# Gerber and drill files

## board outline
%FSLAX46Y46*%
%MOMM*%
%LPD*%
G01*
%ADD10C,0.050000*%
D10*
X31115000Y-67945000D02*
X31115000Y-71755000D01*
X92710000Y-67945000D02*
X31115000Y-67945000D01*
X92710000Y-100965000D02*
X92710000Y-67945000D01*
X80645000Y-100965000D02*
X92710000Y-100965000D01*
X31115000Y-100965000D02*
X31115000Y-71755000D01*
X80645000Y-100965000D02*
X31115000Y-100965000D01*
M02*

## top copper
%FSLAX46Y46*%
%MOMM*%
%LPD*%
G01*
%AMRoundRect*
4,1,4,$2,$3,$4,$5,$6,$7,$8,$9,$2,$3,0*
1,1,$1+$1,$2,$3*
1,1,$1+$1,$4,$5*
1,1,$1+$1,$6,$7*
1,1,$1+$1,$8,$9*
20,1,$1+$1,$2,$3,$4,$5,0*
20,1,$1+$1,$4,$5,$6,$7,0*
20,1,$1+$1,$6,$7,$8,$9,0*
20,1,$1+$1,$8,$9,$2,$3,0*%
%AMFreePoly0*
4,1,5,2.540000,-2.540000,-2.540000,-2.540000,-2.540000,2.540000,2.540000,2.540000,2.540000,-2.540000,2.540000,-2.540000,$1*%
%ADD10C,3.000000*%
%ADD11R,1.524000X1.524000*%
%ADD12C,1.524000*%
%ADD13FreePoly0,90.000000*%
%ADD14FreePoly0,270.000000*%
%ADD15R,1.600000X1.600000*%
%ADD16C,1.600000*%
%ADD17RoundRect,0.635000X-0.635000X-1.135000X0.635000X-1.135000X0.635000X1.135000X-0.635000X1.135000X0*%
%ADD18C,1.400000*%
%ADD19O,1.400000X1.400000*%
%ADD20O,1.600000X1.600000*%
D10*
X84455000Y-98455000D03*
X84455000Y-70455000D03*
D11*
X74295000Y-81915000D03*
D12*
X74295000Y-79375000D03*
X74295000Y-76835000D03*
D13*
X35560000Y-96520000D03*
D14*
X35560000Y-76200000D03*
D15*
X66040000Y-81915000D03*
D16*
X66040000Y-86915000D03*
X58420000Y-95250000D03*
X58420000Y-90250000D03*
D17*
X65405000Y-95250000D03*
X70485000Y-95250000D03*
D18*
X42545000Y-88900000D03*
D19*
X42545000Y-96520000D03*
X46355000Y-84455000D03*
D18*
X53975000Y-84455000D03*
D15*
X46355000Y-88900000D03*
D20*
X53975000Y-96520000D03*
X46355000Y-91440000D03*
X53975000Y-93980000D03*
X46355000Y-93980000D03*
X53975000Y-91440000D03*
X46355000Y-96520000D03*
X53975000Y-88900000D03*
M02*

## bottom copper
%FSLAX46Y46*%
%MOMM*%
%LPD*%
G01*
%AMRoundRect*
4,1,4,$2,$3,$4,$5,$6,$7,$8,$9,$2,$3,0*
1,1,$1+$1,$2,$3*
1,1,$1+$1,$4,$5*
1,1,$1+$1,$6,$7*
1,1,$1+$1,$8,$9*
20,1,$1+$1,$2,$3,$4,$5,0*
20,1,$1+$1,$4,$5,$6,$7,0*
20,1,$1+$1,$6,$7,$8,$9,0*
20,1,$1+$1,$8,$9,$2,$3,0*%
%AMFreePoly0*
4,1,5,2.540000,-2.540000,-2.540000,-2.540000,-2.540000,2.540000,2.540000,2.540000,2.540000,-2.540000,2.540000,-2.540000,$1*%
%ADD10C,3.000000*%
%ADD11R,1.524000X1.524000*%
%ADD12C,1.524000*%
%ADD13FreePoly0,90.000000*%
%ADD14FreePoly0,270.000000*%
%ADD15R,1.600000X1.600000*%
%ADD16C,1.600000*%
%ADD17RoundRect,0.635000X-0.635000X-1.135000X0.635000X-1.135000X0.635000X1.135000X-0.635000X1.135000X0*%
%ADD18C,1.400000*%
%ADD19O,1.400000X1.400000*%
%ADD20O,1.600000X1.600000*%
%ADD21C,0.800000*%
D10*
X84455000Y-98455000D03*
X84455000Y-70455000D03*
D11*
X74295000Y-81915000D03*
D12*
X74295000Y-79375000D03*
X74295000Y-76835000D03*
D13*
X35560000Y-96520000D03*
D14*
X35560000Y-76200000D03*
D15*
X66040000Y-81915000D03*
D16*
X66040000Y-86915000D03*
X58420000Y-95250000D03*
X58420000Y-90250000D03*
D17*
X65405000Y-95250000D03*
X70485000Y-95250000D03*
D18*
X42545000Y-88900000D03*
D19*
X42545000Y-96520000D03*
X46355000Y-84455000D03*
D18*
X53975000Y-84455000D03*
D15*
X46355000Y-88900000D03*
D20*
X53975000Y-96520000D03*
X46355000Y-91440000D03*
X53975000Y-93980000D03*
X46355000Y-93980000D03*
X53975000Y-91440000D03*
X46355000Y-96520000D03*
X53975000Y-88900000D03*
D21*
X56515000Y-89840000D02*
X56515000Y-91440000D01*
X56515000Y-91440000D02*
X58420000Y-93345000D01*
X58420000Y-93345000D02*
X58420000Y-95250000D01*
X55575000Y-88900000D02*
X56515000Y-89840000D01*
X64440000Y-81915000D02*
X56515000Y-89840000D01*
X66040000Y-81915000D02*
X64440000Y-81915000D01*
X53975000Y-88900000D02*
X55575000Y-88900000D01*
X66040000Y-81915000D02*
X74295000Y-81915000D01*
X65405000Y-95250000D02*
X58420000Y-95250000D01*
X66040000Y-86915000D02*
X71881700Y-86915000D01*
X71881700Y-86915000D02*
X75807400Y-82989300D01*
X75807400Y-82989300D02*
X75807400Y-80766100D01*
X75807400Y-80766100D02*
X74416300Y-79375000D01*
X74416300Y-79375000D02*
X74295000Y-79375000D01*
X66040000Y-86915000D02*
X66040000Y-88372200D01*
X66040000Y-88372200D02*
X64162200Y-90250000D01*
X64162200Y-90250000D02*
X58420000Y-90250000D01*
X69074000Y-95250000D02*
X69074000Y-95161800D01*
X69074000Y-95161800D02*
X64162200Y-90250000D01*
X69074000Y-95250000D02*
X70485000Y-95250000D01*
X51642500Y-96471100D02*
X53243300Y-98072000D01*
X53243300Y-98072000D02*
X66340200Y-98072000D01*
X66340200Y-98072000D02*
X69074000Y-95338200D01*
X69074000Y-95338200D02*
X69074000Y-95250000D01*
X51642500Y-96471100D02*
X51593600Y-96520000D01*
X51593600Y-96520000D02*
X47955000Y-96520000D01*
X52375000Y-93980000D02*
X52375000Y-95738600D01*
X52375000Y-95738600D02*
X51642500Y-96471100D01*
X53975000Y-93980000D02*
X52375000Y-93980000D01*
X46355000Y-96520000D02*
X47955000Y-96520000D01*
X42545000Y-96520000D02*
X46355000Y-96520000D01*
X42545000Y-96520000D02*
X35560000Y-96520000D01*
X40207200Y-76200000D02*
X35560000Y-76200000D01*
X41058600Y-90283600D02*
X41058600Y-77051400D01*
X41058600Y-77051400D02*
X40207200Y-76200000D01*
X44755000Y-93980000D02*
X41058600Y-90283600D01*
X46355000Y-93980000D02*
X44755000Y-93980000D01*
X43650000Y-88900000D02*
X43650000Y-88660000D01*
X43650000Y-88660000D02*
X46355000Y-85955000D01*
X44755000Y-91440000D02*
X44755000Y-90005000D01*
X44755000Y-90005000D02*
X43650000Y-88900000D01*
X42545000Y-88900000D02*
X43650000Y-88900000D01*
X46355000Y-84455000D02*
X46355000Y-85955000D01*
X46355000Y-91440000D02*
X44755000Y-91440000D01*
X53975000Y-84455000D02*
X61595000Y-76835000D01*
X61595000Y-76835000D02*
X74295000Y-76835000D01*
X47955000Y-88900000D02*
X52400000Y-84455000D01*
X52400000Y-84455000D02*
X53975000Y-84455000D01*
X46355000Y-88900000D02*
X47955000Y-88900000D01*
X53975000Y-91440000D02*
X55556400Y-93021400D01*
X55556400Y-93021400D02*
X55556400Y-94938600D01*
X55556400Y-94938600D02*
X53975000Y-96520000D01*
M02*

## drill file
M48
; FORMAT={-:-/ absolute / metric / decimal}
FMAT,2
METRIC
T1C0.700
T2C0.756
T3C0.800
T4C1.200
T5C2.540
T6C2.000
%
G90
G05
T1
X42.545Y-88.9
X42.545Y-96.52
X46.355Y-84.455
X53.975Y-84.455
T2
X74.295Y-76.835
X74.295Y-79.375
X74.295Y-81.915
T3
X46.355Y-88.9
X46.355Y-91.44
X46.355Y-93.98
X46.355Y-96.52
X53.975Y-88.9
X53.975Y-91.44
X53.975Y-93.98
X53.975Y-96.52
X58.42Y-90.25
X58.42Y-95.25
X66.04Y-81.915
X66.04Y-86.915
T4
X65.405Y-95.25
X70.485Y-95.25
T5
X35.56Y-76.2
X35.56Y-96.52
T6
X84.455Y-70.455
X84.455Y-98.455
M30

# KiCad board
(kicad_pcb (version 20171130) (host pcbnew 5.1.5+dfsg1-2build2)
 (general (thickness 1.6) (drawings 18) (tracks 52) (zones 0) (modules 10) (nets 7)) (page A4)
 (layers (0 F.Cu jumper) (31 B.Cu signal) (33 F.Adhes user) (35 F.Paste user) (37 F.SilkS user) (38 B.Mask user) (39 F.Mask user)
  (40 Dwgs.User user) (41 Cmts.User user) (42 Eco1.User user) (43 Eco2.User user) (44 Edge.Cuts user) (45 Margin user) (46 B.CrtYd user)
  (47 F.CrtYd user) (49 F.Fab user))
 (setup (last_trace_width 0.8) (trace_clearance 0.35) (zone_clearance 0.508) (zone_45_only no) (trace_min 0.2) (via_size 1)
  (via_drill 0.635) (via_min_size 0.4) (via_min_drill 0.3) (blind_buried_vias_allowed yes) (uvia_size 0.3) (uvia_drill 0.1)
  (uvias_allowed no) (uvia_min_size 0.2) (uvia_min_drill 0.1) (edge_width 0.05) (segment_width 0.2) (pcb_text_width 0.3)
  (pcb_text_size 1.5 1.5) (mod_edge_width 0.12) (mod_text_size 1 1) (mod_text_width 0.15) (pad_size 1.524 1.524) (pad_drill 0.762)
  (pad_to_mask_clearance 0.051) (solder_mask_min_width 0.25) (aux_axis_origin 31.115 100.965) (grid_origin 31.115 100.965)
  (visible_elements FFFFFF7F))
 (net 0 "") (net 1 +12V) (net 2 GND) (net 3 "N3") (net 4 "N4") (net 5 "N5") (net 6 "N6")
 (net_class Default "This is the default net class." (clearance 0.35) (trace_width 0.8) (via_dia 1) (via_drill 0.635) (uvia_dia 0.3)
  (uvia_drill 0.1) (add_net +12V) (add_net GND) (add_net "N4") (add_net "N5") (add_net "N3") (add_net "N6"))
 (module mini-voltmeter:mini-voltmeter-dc (layer F.Cu) (at 84.455 84.455 90)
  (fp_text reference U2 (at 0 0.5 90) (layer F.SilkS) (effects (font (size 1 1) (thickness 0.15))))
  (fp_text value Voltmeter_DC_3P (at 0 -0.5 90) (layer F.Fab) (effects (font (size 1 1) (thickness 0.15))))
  (pad "" np_thru_hole circle (at -14 0 90) (size 3 3) (drill 2) (layers *.Cu *.Mask))
  (pad "" np_thru_hole circle (at 14 0 90) (size 3 3) (drill 2) (layers *.Cu *.Mask))
  (pad 1 thru_hole rect (at 2.54 -10.16 90) (size 1.524 1.524) (drill 0.756) (layers *.Cu *.Mask) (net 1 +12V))
  (pad 2 thru_hole circle (at 5.08 -10.16 90) (size 1.524 1.524) (drill 0.756) (layers *.Cu *.Mask) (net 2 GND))
  (pad 3 thru_hole circle (at 7.62 -10.16 90) (size 1.524 1.524) (drill 0.756) (layers *.Cu *.Mask) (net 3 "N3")))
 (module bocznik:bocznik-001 (layer F.Cu) (at 35.56 86.36 270)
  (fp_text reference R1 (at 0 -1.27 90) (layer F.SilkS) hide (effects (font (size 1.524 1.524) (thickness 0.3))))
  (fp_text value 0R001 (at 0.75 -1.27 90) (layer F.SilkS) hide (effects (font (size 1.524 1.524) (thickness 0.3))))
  (pad 2 thru_hole custom (at 10.16 0 90) (size 5.08 5.08) (drill 2.54) (layers B.Cu B.Mask) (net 2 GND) (zone_connect 0)
   (options (clearance outline) (anchor rect)) (primitives))
  (pad 1 thru_hole custom (at -10.16 0 270) (size 5.08 5.08) (drill 2.54) (layers B.Cu B.Mask) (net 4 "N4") (zone_connect 0)
   (options (clearance outline) (anchor rect)) (primitives)))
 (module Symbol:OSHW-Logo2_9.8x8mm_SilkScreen (layer F.Cu) (at 50.165 76.835)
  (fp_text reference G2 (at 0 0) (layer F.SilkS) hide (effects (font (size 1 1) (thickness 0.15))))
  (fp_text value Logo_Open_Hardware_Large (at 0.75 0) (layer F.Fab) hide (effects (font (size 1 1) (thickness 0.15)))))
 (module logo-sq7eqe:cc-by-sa (layer F.Cu) (at 62.865 76.2)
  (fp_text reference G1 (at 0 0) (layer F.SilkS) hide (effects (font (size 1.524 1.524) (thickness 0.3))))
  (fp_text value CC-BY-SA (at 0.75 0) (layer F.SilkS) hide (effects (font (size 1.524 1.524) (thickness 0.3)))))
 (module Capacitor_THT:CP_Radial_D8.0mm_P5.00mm (layer F.Cu) (at 66.04 81.915 270)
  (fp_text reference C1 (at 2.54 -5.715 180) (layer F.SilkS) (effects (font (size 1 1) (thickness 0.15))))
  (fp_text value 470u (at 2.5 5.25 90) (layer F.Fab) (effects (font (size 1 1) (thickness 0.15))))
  (pad 1 thru_hole rect (at 0 0 270) (size 1.6 1.6) (drill 0.8) (layers *.Cu *.Mask) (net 1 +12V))
  (pad 2 thru_hole circle (at 5 0 270) (size 1.6 1.6) (drill 0.8) (layers *.Cu *.Mask) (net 2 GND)))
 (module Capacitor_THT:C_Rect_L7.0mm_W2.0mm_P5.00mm (layer F.Cu) (at 58.42 95.25 90)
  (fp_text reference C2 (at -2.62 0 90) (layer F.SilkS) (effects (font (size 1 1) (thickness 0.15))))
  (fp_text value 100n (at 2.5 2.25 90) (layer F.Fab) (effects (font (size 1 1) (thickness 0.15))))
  (pad 1 thru_hole circle (at 0 0 90) (size 1.6 1.6) (drill 0.8) (layers *.Cu *.Mask) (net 1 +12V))
  (pad 2 thru_hole circle (at 5 0 90) (size 1.6 1.6) (drill 0.8) (layers *.Cu *.Mask) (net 2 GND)))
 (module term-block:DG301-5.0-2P (layer F.Cu) (at 67.905 95.25)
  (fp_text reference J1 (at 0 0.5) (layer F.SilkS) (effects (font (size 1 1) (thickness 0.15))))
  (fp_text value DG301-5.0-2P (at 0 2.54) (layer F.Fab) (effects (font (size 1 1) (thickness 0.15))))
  (pad 1 thru_hole roundrect (at -2.5 0) (size 2.54 3.54) (drill 1.2) (layers *.Cu *.Mask) (roundrect_rratio 0.25) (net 1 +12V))
  (pad 2 thru_hole roundrect (at 2.58 0) (size 2.54 3.54) (drill 1.2) (layers *.Cu *.Mask) (roundrect_rratio 0.25) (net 2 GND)))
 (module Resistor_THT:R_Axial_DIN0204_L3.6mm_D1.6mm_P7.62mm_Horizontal (layer F.Cu) (at 42.545 88.9 270)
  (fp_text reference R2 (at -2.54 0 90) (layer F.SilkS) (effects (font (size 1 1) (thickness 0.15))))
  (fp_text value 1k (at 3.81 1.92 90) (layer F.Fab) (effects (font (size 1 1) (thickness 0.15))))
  (pad 1 thru_hole circle (at 0 0 270) (size 1.4 1.4) (drill 0.7) (layers *.Cu *.Mask) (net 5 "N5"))
  (pad 2 thru_hole oval (at 7.62 0 270) (size 1.4 1.4) (drill 0.7) (layers *.Cu *.Mask) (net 2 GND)))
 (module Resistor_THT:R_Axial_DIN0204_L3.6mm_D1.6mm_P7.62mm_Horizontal (layer F.Cu) (at 53.975 84.455 180)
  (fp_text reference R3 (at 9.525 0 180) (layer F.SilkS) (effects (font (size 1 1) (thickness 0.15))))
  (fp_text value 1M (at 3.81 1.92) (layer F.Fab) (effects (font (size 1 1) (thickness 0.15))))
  (pad 2 thru_hole oval (at 7.62 0 180) (size 1.4 1.4) (drill 0.7) (layers *.Cu *.Mask) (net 5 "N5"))
  (pad 1 thru_hole circle (at 0 0 180) (size 1.4 1.4) (drill 0.7) (layers *.Cu *.Mask) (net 3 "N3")))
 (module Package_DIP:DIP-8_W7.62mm (layer F.Cu) (at 46.355 88.9)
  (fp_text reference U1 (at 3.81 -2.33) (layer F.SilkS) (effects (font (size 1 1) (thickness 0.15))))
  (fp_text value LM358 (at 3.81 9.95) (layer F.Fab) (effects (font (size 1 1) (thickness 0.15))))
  (pad 1 thru_hole rect (at 0 0) (size 1.6 1.6) (drill 0.8) (layers *.Cu *.Mask) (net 3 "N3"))
  (pad 5 thru_hole oval (at 7.62 7.62) (size 1.6 1.6) (drill 0.8) (layers *.Cu *.Mask) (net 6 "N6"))
  (pad 2 thru_hole oval (at 0 2.54) (size 1.6 1.6) (drill 0.8) (layers *.Cu *.Mask) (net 5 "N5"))
  (pad 6 thru_hole oval (at 7.62 5.08) (size 1.6 1.6) (drill 0.8) (layers *.Cu *.Mask) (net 2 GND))
  (pad 3 thru_hole oval (at 0 5.08) (size 1.6 1.6) (drill 0.8) (layers *.Cu *.Mask) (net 4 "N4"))
  (pad 7 thru_hole oval (at 7.62 2.54) (size 1.6 1.6) (drill 0.8) (layers *.Cu *.Mask) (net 6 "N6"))
  (pad 4 thru_hole oval (at 0 7.62) (size 1.6 1.6) (drill 0.8) (layers *.Cu *.Mask) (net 2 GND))
  (pad 8 thru_hole oval (at 7.62 0) (size 1.6 1.6) (drill 0.8) (layers *.Cu *.Mask) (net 1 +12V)))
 (gr_line (start 31.115 67.945) (end 31.115 71.755) (layer Edge.Cuts) (width 0.05))
 (gr_line (start 92.71 67.945) (end 31.115 67.945) (layer Edge.Cuts) (width 0.05))
 (gr_line (start 92.71 100.965) (end 92.71 67.945) (layer Edge.Cuts) (width 0.05))
 (gr_line (start 80.645 100.965) (end 92.71 100.965) (layer Edge.Cuts) (width 0.05))
 (gr_line (start 31.115 100.965) (end 31.115 71.755) (layer Edge.Cuts) (width 0.05))
 (gr_line (start 80.645 100.965) (end 31.115 100.965) (layer Edge.Cuts) (width 0.05))
 (segment (start 56.515 89.84) (end 56.515 91.44) (width 0.8) (layer B.Cu) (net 1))
 (segment (start 56.515 91.44) (end 58.42 93.345) (width 0.8) (layer B.Cu) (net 1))
 (segment (start 58.42 93.345) (end 58.42 95.25) (width 0.8) (layer B.Cu) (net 1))
 (segment (start 55.575 88.9) (end 56.515 89.84) (width 0.8) (layer B.Cu) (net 1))
 (segment (start 64.44 81.915) (end 56.515 89.84) (width 0.8) (layer B.Cu) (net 1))
 (segment (start 66.04 81.915) (end 64.44 81.915) (width 0.8) (layer B.Cu) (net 1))
 (segment (start 53.975 88.9) (end 55.575 88.9) (width 0.8) (layer B.Cu) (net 1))
 (segment (start 66.04 81.915) (end 74.295 81.915) (width 0.8) (layer B.Cu) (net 1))
 (segment (start 65.405 95.25) (end 58.42 95.25) (width 0.8) (layer B.Cu) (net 1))
 (segment (start 66.04 86.915) (end 71.8817 86.915) (width 0.8) (layer B.Cu) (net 2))
 (segment (start 71.8817 86.915) (end 75.8074 82.9893) (width 0.8) (layer B.Cu) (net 2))
 (segment (start 75.8074 82.9893) (end 75.8074 80.7661) (width 0.8) (layer B.Cu) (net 2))
 (segment (start 75.8074 80.7661) (end 74.4163 79.375) (width 0.8) (layer B.Cu) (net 2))
 (segment (start 74.4163 79.375) (end 74.295 79.375) (width 0.8) (layer B.Cu) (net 2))
 (segment (start 66.04 86.915) (end 66.04 88.3722) (width 0.8) (layer B.Cu) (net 2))
 (segment (start 66.04 88.3722) (end 64.1622 90.25) (width 0.8) (layer B.Cu) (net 2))
 (segment (start 64.1622 90.25) (end 58.42 90.25) (width 0.8) (layer B.Cu) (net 2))
 (segment (start 69.074 95.25) (end 69.074 95.1618) (width 0.8) (layer B.Cu) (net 2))
 (segment (start 69.074 95.1618) (end 64.1622 90.25) (width 0.8) (layer B.Cu) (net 2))
 (segment (start 69.074 95.25) (end 70.485 95.25) (width 0.8) (layer B.Cu) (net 2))
 (segment (start 51.6425 96.4711) (end 53.2433 98.072) (width 0.8) (layer B.Cu) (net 2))
 (segment (start 53.2433 98.072) (end 66.3402 98.072) (width 0.8) (layer B.Cu) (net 2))
 (segment (start 66.3402 98.072) (end 69.074 95.3382) (width 0.8) (layer B.Cu) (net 2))
 (segment (start 69.074 95.3382) (end 69.074 95.25) (width 0.8) (layer B.Cu) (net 2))
 (segment (start 51.6425 96.4711) (end 51.5936 96.52) (width 0.8) (layer B.Cu) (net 2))
 (segment (start 51.5936 96.52) (end 47.955 96.52) (width 0.8) (layer B.Cu) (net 2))
 (segment (start 52.375 93.98) (end 52.375 95.7386) (width 0.8) (layer B.Cu) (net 2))
 (segment (start 52.375 95.7386) (end 51.6425 96.4711) (width 0.8) (layer B.Cu) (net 2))
 (segment (start 53.975 93.98) (end 52.375 93.98) (width 0.8) (layer B.Cu) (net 2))
 (segment (start 46.355 96.52) (end 47.955 96.52) (width 0.8) (layer B.Cu) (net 2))
 (segment (start 42.545 96.52) (end 46.355 96.52) (width 0.8) (layer B.Cu) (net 2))
 (segment (start 42.545 96.52) (end 35.56 96.52) (width 0.8) (layer B.Cu) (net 2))
 (segment (start 40.2072 76.2) (end 35.56 76.2) (width 0.8) (layer B.Cu) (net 4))
 (segment (start 41.0586 90.2836) (end 41.0586 77.0514) (width 0.8) (layer B.Cu) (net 4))
 (segment (start 41.0586 77.0514) (end 40.2072 76.2) (width 0.8) (layer B.Cu) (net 4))
 (segment (start 44.755 93.98) (end 41.0586 90.2836) (width 0.8) (layer B.Cu) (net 4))
 (segment (start 46.355 93.98) (end 44.755 93.98) (width 0.8) (layer B.Cu) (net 4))
 (segment (start 43.65 88.9) (end 43.65 88.66) (width 0.8) (layer B.Cu) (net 5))
 (segment (start 43.65 88.66) (end 46.355 85.955) (width 0.8) (layer B.Cu) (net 5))
 (segment (start 44.755 91.44) (end 44.755 90.005) (width 0.8) (layer B.Cu) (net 5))
 (segment (start 44.755 90.005) (end 43.65 88.9) (width 0.8) (layer B.Cu) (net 5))
 (segment (start 42.545 88.9) (end 43.65 88.9) (width 0.8) (layer B.Cu) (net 5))
 (segment (start 46.355 84.455) (end 46.355 85.955) (width 0.8) (layer B.Cu) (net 5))
 (segment (start 46.355 91.44) (end 44.755 91.44) (width 0.8) (layer B.Cu) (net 5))
 (segment (start 53.975 84.455) (end 61.595 76.835) (width 0.8) (layer B.Cu) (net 3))
 (segment (start 61.595 76.835) (end 74.295 76.835) (width 0.8) (layer B.Cu) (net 3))
 (segment (start 47.955 88.9) (end 52.4 84.455) (width 0.8) (layer B.Cu) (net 3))
 (segment (start 52.4 84.455) (end 53.975 84.455) (width 0.8) (layer B.Cu) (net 3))
 (segment (start 46.355 88.9) (end 47.955 88.9) (width 0.8) (layer B.Cu) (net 3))
 (segment (start 53.975 91.44) (end 55.5564 93.0214) (width 0.8) (layer B.Cu) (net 6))
 (segment (start 55.5564 93.0214) (end 55.5564 94.9386) (width 0.8) (layer B.Cu) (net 6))
 (segment (start 55.5564 94.9386) (end 53.975 96.52) (width 0.8) (layer B.Cu) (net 6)))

